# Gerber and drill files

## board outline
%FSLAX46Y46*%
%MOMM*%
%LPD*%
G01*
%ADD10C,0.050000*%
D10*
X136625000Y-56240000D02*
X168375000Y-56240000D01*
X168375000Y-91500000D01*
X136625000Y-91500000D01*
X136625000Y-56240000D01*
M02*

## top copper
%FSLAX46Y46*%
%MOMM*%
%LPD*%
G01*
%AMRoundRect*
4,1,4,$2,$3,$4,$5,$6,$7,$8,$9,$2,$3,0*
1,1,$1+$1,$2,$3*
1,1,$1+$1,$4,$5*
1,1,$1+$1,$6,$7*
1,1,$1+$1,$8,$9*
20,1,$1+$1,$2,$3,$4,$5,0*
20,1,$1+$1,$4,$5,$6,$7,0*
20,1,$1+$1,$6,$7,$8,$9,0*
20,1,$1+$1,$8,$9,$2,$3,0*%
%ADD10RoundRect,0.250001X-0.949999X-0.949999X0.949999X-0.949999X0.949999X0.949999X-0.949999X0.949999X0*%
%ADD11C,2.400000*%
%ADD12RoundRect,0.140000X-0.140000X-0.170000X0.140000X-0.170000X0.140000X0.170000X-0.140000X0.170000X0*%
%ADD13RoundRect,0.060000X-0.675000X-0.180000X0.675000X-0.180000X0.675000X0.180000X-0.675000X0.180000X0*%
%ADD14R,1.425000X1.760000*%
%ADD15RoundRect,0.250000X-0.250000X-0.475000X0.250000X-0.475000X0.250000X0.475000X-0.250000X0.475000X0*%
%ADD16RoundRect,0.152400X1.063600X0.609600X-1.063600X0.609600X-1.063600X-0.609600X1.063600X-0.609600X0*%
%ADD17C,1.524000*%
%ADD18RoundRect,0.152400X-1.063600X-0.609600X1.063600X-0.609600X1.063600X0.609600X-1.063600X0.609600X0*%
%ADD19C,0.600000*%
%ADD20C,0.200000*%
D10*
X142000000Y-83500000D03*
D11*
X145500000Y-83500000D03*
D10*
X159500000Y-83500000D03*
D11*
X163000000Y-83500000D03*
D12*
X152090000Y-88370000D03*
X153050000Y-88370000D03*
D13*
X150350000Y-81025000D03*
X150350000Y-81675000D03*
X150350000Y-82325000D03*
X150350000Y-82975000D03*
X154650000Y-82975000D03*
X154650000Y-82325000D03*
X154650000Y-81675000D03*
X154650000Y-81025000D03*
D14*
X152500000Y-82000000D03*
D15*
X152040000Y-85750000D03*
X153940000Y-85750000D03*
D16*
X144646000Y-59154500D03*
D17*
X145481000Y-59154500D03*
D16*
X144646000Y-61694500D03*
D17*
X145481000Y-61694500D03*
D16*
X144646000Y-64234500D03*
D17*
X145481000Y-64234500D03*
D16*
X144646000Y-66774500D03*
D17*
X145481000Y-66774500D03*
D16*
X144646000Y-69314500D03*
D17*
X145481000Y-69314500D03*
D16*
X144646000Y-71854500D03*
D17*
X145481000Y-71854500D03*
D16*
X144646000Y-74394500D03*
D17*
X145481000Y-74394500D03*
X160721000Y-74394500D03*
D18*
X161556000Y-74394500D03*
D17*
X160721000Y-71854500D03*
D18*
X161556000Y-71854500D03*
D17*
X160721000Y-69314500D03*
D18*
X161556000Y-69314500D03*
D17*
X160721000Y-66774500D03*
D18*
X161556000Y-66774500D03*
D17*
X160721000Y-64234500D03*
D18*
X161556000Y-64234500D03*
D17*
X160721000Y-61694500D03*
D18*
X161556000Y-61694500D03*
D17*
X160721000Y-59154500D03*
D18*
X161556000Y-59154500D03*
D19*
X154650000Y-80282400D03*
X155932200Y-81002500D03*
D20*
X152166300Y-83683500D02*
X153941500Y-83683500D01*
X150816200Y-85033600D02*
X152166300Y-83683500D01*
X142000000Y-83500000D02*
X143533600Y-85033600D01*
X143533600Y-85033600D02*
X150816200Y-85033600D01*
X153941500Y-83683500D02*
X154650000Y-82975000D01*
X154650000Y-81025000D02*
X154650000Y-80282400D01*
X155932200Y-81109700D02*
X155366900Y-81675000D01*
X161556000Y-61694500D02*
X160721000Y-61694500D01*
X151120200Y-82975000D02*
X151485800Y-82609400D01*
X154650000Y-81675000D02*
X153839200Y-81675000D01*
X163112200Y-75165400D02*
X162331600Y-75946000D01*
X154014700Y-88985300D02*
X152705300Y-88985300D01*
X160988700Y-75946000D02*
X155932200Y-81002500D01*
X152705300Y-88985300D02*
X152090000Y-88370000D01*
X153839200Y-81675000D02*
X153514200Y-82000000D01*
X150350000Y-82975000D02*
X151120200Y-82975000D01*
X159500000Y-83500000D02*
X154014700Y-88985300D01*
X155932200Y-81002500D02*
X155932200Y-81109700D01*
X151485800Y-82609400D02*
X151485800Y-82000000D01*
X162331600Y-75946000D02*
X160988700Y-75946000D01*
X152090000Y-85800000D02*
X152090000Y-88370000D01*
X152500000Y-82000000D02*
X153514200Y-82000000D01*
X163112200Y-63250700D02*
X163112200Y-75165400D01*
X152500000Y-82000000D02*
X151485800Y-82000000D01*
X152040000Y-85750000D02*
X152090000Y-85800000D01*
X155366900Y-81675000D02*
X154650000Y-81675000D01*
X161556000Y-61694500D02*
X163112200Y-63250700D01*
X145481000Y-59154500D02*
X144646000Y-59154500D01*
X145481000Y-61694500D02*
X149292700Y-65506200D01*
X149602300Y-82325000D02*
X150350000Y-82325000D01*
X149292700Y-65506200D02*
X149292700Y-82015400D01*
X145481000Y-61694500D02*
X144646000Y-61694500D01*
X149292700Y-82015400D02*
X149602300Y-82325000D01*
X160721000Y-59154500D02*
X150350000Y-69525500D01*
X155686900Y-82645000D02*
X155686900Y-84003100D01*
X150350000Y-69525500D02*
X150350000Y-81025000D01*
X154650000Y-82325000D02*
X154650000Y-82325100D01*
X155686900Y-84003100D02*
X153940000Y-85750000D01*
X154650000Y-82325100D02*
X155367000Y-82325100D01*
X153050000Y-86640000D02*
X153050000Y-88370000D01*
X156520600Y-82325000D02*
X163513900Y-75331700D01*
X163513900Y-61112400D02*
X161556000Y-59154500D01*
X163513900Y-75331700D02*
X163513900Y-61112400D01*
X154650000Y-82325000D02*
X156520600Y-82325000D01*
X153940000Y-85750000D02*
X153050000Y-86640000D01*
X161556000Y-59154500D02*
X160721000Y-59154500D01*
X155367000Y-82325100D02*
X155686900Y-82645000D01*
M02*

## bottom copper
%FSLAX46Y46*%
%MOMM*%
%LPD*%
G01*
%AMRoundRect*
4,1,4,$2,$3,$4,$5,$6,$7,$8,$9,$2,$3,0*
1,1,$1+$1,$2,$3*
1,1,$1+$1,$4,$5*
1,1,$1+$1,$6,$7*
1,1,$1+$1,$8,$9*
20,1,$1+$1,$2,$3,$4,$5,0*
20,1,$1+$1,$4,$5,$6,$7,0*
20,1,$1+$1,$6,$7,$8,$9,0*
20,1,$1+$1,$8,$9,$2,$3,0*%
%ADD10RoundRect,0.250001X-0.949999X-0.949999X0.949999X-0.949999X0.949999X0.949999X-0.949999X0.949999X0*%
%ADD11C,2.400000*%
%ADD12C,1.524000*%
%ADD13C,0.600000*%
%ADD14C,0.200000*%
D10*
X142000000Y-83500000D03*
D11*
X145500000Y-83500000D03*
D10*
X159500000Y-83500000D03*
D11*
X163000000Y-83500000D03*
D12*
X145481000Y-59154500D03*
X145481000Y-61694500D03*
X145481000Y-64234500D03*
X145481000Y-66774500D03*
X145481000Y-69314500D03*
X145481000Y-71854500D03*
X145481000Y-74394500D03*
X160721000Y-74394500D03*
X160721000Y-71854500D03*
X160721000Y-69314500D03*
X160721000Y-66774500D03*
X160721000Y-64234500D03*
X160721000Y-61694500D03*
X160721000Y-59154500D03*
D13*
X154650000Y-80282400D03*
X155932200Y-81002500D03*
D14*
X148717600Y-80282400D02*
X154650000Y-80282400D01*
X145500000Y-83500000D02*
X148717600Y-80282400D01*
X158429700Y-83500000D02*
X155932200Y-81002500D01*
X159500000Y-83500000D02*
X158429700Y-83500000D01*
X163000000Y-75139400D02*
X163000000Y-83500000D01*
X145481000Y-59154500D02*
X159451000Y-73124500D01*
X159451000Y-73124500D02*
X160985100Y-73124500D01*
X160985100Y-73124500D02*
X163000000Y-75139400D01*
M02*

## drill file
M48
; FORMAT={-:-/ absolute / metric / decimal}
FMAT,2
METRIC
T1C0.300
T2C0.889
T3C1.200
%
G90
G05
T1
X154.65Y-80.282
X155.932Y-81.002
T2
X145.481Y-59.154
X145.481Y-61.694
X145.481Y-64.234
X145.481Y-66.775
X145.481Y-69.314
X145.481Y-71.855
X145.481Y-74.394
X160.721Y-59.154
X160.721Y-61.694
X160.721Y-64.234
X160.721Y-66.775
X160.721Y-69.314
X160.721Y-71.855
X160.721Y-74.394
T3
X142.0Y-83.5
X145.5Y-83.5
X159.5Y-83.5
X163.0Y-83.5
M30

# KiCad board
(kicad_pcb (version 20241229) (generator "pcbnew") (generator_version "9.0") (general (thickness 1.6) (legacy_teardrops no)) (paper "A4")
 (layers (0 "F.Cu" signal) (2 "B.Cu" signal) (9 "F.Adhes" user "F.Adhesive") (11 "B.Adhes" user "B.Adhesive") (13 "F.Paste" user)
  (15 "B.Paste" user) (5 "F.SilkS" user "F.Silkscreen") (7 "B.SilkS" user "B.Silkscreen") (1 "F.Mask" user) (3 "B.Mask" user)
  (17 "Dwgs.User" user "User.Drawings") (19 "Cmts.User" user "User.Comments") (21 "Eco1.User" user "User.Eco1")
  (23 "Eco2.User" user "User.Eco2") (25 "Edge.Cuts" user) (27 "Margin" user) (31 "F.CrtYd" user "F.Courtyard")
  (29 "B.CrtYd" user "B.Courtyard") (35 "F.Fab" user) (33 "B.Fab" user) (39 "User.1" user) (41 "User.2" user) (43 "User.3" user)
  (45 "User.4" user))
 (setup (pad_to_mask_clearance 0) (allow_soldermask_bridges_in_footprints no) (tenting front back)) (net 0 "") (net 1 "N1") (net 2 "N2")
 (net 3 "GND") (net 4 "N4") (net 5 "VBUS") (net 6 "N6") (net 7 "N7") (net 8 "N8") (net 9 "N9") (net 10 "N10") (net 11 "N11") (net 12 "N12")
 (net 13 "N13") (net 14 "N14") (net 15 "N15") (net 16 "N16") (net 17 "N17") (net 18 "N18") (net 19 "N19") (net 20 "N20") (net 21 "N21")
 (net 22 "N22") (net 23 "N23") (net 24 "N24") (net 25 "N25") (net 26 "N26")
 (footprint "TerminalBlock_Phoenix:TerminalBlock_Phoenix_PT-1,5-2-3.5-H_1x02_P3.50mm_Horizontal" (layer "F.Cu") (at 142 83.5)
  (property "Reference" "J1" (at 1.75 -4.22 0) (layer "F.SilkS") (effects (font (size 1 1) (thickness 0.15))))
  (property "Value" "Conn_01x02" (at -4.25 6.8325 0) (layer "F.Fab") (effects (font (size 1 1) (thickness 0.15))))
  (pad "1" thru_hole roundrect (at 0 0) (size 2.4 2.4) (drill 1.2) (layers "*.Cu" "*.Mask") (remove_unused_layers no)
   (roundrect_rratio 0.104167) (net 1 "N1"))
  (pad "2" thru_hole circle (at 3.5 0) (size 2.4 2.4) (drill 1.2) (layers "*.Cu" "*.Mask") (remove_unused_layers no) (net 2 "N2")))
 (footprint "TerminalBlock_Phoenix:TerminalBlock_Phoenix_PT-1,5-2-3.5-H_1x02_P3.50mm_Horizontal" (layer "F.Cu") (at 159.5 83.5)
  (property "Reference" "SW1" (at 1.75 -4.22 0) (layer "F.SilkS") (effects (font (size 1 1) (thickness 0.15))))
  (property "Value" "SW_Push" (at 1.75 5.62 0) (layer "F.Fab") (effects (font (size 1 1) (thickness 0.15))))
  (pad "1" thru_hole roundrect (at 0 0) (size 2.4 2.4) (drill 1.2) (layers "*.Cu" "*.Mask") (remove_unused_layers no)
   (roundrect_rratio 0.104167) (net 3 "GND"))
  (pad "2" thru_hole circle (at 3.5 0) (size 2.4 2.4) (drill 1.2) (layers "*.Cu" "*.Mask") (remove_unused_layers no) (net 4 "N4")))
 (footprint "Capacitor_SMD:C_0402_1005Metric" (layer "F.Cu") (at 152.57 88.37)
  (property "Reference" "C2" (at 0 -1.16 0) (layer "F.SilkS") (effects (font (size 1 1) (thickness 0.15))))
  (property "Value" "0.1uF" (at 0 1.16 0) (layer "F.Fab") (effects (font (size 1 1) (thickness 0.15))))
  (pad "1" smd roundrect (at -0.48 0) (size 0.56 0.62) (layers "F.Cu" "F.Mask" "F.Paste") (roundrect_rratio 0.25) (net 3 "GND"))
  (pad "2" smd roundrect (at 0.48 0) (size 0.56 0.62) (layers "F.Cu" "F.Mask" "F.Paste") (roundrect_rratio 0.25) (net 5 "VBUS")))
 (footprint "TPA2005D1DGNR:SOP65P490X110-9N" (layer "F.Cu") (at 152.5 82)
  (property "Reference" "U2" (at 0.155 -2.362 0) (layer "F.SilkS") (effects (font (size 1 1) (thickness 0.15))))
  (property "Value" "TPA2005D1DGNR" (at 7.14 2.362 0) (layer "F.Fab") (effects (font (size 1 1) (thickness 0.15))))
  (pad "1" smd roundrect (at -2.15 -0.975) (size 1.47 0.48) (layers "F.Cu" "F.Mask" "F.Paste") (roundrect_rratio 0.125) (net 5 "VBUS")
   (solder_mask_margin 0.102))
  (pad "2" smd roundrect (at -2.15 -0.325) (size 1.47 0.48) (layers "F.Cu" "F.Mask" "F.Paste") (roundrect_rratio 0.125)
   (solder_mask_margin 0.102))
  (pad "3" smd roundrect (at -2.15 0.325) (size 1.47 0.48) (layers "F.Cu" "F.Mask" "F.Paste") (roundrect_rratio 0.125) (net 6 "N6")
   (solder_mask_margin 0.102))
  (pad "4" smd roundrect (at -2.15 0.975) (size 1.47 0.48) (layers "F.Cu" "F.Mask" "F.Paste") (roundrect_rratio 0.125) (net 3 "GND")
   (solder_mask_margin 0.102))
  (pad "5" smd roundrect (at 2.15 0.975) (size 1.47 0.48) (layers "F.Cu" "F.Mask" "F.Paste") (roundrect_rratio 0.125) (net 1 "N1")
   (solder_mask_margin 0.102))
  (pad "6" smd roundrect (at 2.15 0.325) (size 1.47 0.48) (layers "F.Cu" "F.Mask" "F.Paste") (roundrect_rratio 0.125) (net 5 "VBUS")
   (solder_mask_margin 0.102))
  (pad "7" smd roundrect (at 2.15 -0.325) (size 1.47 0.48) (layers "F.Cu" "F.Mask" "F.Paste") (roundrect_rratio 0.125) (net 3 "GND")
   (solder_mask_margin 0.102))
  (pad "8" smd roundrect (at 2.15 -0.975) (size 1.47 0.48) (layers "F.Cu" "F.Mask" "F.Paste") (roundrect_rratio 0.125) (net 2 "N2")
   (solder_mask_margin 0.102))
  (pad "9" smd rect (at 0 0) (size 1.425 1.76) (layers "F.Cu" "F.Mask") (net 3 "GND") (solder_mask_margin 0.102)))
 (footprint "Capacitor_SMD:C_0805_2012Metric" (layer "F.Cu") (at 152.99 85.75)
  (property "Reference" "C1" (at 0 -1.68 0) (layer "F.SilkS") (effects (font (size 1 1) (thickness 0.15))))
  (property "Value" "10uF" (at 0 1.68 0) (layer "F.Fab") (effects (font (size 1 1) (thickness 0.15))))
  (pad "1" smd roundrect (at -0.95 0) (size 1 1.45) (layers "F.Cu" "F.Mask" "F.Paste") (roundrect_rratio 0.25) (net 3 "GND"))
  (pad "2" smd roundrect (at 0.95 0) (size 1 1.45) (layers "F.Cu" "F.Mask" "F.Paste") (roundrect_rratio 0.25) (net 5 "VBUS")))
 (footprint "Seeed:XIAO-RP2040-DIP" (layer "F.Cu") (at 153.101 66.7745)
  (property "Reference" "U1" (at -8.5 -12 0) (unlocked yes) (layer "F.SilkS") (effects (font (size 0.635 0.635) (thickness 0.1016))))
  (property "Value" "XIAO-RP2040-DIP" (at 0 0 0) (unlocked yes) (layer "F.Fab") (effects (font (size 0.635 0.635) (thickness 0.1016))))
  (pad "1" smd roundrect (at -8.455 -7.62 180) (size 2.432 1.524) (layers "F.Cu" "F.Mask") (roundrect_rratio 0.1) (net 4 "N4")
   (thermal_bridge_angle 45))
  (pad "1" thru_hole circle (at -7.62 -7.62 180) (size 1.524 1.524) (drill 0.889) (layers "*.Cu" "*.Mask") (remove_unused_layers no)
   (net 4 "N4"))
  (pad "2" smd roundrect (at -8.455 -5.08 180) (size 2.432 1.524) (layers "F.Cu" "F.Mask") (roundrect_rratio 0.1) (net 6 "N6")
   (thermal_bridge_angle 45))
  (pad "2" thru_hole circle (at -7.62 -5.08 180) (size 1.524 1.524) (drill 0.889) (layers "*.Cu" "*.Mask") (remove_unused_layers no)
   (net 6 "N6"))
  (pad "3" smd roundrect (at -8.455 -2.54 180) (size 2.432 1.524) (layers "F.Cu" "F.Mask") (roundrect_rratio 0.1) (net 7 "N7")
   (thermal_bridge_angle 45))
  (pad "3" thru_hole circle (at -7.62 -2.54 180) (size 1.524 1.524) (drill 0.889) (layers "*.Cu" "*.Mask") (remove_unused_layers no)
   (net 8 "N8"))
  (pad "4" smd roundrect (at -8.455 0 180) (size 2.432 1.524) (layers "F.Cu" "F.Mask") (roundrect_rratio 0.1) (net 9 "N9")
   (thermal_bridge_angle 45))
  (pad "4" thru_hole circle (at -7.62 0 180) (size 1.524 1.524) (drill 0.889) (layers "*.Cu" "*.Mask") (remove_unused_layers no)
   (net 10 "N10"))
  (pad "5" smd roundrect (at -8.455 2.54 180) (size 2.432 1.524) (layers "F.Cu" "F.Mask") (roundrect_rratio 0.1) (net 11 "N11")
   (thermal_bridge_angle 45))
  (pad "5" thru_hole circle (at -7.62 2.54 180) (size 1.524 1.524) (drill 0.889) (layers "*.Cu" "*.Mask") (remove_unused_layers no)
   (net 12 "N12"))
  (pad "6" smd roundrect (at -8.455 5.08 180) (size 2.432 1.524) (layers "F.Cu" "F.Mask") (roundrect_rratio 0.1) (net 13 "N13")
   (thermal_bridge_angle 45))
  (pad "6" thru_hole circle (at -7.62 5.08 180) (size 1.524 1.524) (drill 0.889) (layers "*.Cu" "*.Mask") (remove_unused_layers no)
   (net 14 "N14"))
  (pad "7" smd roundrect (at -8.455 7.62 180) (size 2.432 1.524) (layers "F.Cu" "F.Mask") (roundrect_rratio 0.1) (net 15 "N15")
   (thermal_bridge_angle 45))
  (pad "7" thru_hole circle (at -7.62 7.62 180) (size 1.524 1.524) (drill 0.889) (layers "*.Cu" "*.Mask") (remove_unused_layers no)
   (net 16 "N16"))
  (pad "8" thru_hole circle (at 7.62 7.62) (size 1.524 1.524) (drill 0.889) (layers "*.Cu" "*.Mask") (remove_unused_layers no)
   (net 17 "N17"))
  (pad "8" smd roundrect (at 8.455 7.62) (size 2.432 1.524) (layers "F.Cu" "F.Mask") (roundrect_rratio 0.1) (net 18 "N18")
   (thermal_bridge_angle 45))
  (pad "9" thru_hole circle (at 7.62 5.08) (size 1.524 1.524) (drill 0.889) (layers "*.Cu" "*.Mask") (remove_unused_layers no)
   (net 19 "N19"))
  (pad "9" smd roundrect (at 8.455 5.08) (size 2.432 1.524) (layers "F.Cu" "F.Mask") (roundrect_rratio 0.1) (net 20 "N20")
   (thermal_bridge_angle 45))
  (pad "10" thru_hole circle (at 7.62 2.54) (size 1.524 1.524) (drill 0.889) (layers "*.Cu" "*.Mask") (remove_unused_layers no)
   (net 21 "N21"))
  (pad "10" smd roundrect (at 8.455 2.54) (size 2.432 1.524) (layers "F.Cu" "F.Mask") (roundrect_rratio 0.1) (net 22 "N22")
   (thermal_bridge_angle 45))
  (pad "11" thru_hole circle (at 7.62 0) (size 1.524 1.524) (drill 0.889) (layers "*.Cu" "*.Mask") (remove_unused_layers no) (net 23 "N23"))
  (pad "11" smd roundrect (at 8.455 0) (size 2.432 1.524) (layers "F.Cu" "F.Mask") (roundrect_rratio 0.1) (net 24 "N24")
   (thermal_bridge_angle 45))
  (pad "12" thru_hole circle (at 7.62 -2.54) (size 1.524 1.524) (drill 0.889) (layers "*.Cu" "*.Mask") (remove_unused_layers no)
   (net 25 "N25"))
  (pad "12" smd roundrect (at 8.455 -2.54) (size 2.432 1.524) (layers "F.Cu" "F.Mask") (roundrect_rratio 0.1) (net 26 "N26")
   (thermal_bridge_angle 45))
  (pad "13" thru_hole circle (at 7.62 -5.08) (size 1.524 1.524) (drill 0.889) (layers "*.Cu" "*.Mask") (remove_unused_layers no)
   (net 3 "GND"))
  (pad "13" smd roundrect (at 8.455 -5.08) (size 2.432 1.524) (layers "F.Cu" "F.Mask") (roundrect_rratio 0.1) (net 3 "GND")
   (thermal_bridge_angle 45))
  (pad "14" thru_hole circle (at 7.62 -7.62) (size 1.524 1.524) (drill 0.889) (layers "*.Cu" "*.Mask") (remove_unused_layers no)
   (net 5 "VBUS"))
  (pad "14" smd roundrect (at 8.455 -7.62) (size 2.432 1.524) (layers "F.Cu" "F.Mask") (roundrect_rratio 0.1) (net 5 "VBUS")
   (thermal_bridge_angle 45)))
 (gr_rect (start 136.625 56.24) (end 168.375 91.5) (stroke (width 0.05) (type default)) (fill no) (layer "Edge.Cuts"))
 (segment (start 152.1663 83.6835) (end 153.9415 83.6835) (width 0.2) (layer "F.Cu") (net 1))
 (segment (start 150.8162 85.0336) (end 152.1663 83.6835) (width 0.2) (layer "F.Cu") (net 1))
 (segment (start 142 83.5) (end 143.5336 85.0336) (width 0.2) (layer "F.Cu") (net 1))
 (segment (start 143.5336 85.0336) (end 150.8162 85.0336) (width 0.2) (layer "F.Cu") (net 1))
 (segment (start 153.9415 83.6835) (end 154.65 82.975) (width 0.2) (layer "F.Cu") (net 1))
 (segment (start 154.65 81.025) (end 154.65 80.2824) (width 0.2) (layer "F.Cu") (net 2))
 (via (at 154.65 80.2824) (size 0.6) (drill 0.3) (layers "F.Cu" "B.Cu") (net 2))
 (segment (start 148.7176 80.2824) (end 154.65 80.2824) (width 0.2) (layer "B.Cu") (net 2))
 (segment (start 145.5 83.5) (end 148.7176 80.2824) (width 0.2) (layer "B.Cu") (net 2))
 (segment (start 155.9322 81.1097) (end 155.3669 81.675) (width 0.2) (layer "F.Cu") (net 3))
 (segment (start 161.556 61.6945) (end 160.721 61.6945) (width 0.2) (layer "F.Cu") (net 3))
 (segment (start 151.1202 82.975) (end 151.4858 82.6094) (width 0.2) (layer "F.Cu") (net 3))
 (segment (start 154.65 81.675) (end 153.8392 81.675) (width 0.2) (layer "F.Cu") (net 3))
 (segment (start 163.1122 75.1654) (end 162.3316 75.946) (width 0.2) (layer "F.Cu") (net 3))
 (segment (start 154.0147 88.9853) (end 152.7053 88.9853) (width 0.2) (layer "F.Cu") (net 3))
 (segment (start 160.9887 75.946) (end 155.9322 81.0025) (width 0.2) (layer "F.Cu") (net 3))
 (segment (start 152.7053 88.9853) (end 152.09 88.37) (width 0.2) (layer "F.Cu") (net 3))
 (segment (start 153.8392 81.675) (end 153.5142 82) (width 0.2) (layer "F.Cu") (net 3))
 (segment (start 150.35 82.975) (end 151.1202 82.975) (width 0.2) (layer "F.Cu") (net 3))
 (segment (start 159.5 83.5) (end 154.0147 88.9853) (width 0.2) (layer "F.Cu") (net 3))
 (segment (start 155.9322 81.0025) (end 155.9322 81.1097) (width 0.2) (layer "F.Cu") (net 3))
 (segment (start 151.4858 82.6094) (end 151.4858 82) (width 0.2) (layer "F.Cu") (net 3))
 (segment (start 162.3316 75.946) (end 160.9887 75.946) (width 0.2) (layer "F.Cu") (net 3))
 (segment (start 152.09 85.8) (end 152.09 88.37) (width 0.2) (layer "F.Cu") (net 3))
 (segment (start 152.5 82) (end 153.5142 82) (width 0.2) (layer "F.Cu") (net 3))
 (segment (start 163.1122 63.2507) (end 163.1122 75.1654) (width 0.2) (layer "F.Cu") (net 3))
 (segment (start 152.5 82) (end 151.4858 82) (width 0.2) (layer "F.Cu") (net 3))
 (segment (start 152.04 85.75) (end 152.09 85.8) (width 0.2) (layer "F.Cu") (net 3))
 (segment (start 155.3669 81.675) (end 154.65 81.675) (width 0.2) (layer "F.Cu") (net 3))
 (segment (start 161.556 61.6945) (end 163.1122 63.2507) (width 0.2) (layer "F.Cu") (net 3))
 (via (at 155.9322 81.0025) (size 0.6) (drill 0.3) (layers "F.Cu" "B.Cu") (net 3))
 (segment (start 158.4297 83.5) (end 155.9322 81.0025) (width 0.2) (layer "B.Cu") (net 3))
 (segment (start 159.5 83.5) (end 158.4297 83.5) (width 0.2) (layer "B.Cu") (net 3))
 (segment (start 145.481 59.1545) (end 144.646 59.1545) (width 0.2) (layer "F.Cu") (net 4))
 (segment (start 163 75.1394) (end 163 83.5) (width 0.2) (layer "B.Cu") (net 4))
 (segment (start 145.481 59.1545) (end 159.451 73.1245) (width 0.2) (layer "B.Cu") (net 4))
 (segment (start 159.451 73.1245) (end 160.9851 73.1245) (width 0.2) (layer "B.Cu") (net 4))
 (segment (start 160.9851 73.1245) (end 163 75.1394) (width 0.2) (layer "B.Cu") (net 4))
 (segment (start 145.481 61.6945) (end 149.2927 65.5062) (width 0.2) (layer "F.Cu") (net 6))
 (segment (start 149.6023 82.325) (end 150.35 82.325) (width 0.2) (layer "F.Cu") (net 6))
 (segment (start 149.2927 65.5062) (end 149.2927 82.0154) (width 0.2) (layer "F.Cu") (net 6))
 (segment (start 145.481 61.6945) (end 144.646 61.6945) (width 0.2) (layer "F.Cu") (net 6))
 (segment (start 149.2927 82.0154) (end 149.6023 82.325) (width 0.2) (layer "F.Cu") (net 6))
 (segment (start 160.721 59.1545) (end 150.35 69.5255) (width 0.2) (layer "F.Cu") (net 5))
 (segment (start 155.6869 82.645) (end 155.6869 84.0031) (width 0.2) (layer "F.Cu") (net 5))
 (segment (start 150.35 69.5255) (end 150.35 81.025) (width 0.2) (layer "F.Cu") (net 5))
 (segment (start 154.65 82.325) (end 154.65 82.3251) (width 0.2) (layer "F.Cu") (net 5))
 (segment (start 155.6869 84.0031) (end 153.94 85.75) (width 0.2) (layer "F.Cu") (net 5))
 (segment (start 154.65 82.3251) (end 155.367 82.3251) (width 0.2) (layer "F.Cu") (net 5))
 (segment (start 153.05 86.64) (end 153.05 88.37) (width 0.2) (layer "F.Cu") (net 5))
 (segment (start 156.5206 82.325) (end 163.5139 75.3317) (width 0.2) (layer "F.Cu") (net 5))
 (segment (start 163.5139 61.1124) (end 161.556 59.1545) (width 0.2) (layer "F.Cu") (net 5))
 (segment (start 163.5139 75.3317) (end 163.5139 61.1124) (width 0.2) (layer "F.Cu") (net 5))
 (segment (start 154.65 82.325) (end 156.5206 82.325) (width 0.2) (layer "F.Cu") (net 5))
 (segment (start 153.94 85.75) (end 153.05 86.64) (width 0.2) (layer "F.Cu") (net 5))
 (segment (start 161.556 59.1545) (end 160.721 59.1545) (width 0.2) (layer "F.Cu") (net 5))
 (segment (start 155.367 82.3251) (end 155.6869 82.645) (width 0.2) (layer "F.Cu") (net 5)))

